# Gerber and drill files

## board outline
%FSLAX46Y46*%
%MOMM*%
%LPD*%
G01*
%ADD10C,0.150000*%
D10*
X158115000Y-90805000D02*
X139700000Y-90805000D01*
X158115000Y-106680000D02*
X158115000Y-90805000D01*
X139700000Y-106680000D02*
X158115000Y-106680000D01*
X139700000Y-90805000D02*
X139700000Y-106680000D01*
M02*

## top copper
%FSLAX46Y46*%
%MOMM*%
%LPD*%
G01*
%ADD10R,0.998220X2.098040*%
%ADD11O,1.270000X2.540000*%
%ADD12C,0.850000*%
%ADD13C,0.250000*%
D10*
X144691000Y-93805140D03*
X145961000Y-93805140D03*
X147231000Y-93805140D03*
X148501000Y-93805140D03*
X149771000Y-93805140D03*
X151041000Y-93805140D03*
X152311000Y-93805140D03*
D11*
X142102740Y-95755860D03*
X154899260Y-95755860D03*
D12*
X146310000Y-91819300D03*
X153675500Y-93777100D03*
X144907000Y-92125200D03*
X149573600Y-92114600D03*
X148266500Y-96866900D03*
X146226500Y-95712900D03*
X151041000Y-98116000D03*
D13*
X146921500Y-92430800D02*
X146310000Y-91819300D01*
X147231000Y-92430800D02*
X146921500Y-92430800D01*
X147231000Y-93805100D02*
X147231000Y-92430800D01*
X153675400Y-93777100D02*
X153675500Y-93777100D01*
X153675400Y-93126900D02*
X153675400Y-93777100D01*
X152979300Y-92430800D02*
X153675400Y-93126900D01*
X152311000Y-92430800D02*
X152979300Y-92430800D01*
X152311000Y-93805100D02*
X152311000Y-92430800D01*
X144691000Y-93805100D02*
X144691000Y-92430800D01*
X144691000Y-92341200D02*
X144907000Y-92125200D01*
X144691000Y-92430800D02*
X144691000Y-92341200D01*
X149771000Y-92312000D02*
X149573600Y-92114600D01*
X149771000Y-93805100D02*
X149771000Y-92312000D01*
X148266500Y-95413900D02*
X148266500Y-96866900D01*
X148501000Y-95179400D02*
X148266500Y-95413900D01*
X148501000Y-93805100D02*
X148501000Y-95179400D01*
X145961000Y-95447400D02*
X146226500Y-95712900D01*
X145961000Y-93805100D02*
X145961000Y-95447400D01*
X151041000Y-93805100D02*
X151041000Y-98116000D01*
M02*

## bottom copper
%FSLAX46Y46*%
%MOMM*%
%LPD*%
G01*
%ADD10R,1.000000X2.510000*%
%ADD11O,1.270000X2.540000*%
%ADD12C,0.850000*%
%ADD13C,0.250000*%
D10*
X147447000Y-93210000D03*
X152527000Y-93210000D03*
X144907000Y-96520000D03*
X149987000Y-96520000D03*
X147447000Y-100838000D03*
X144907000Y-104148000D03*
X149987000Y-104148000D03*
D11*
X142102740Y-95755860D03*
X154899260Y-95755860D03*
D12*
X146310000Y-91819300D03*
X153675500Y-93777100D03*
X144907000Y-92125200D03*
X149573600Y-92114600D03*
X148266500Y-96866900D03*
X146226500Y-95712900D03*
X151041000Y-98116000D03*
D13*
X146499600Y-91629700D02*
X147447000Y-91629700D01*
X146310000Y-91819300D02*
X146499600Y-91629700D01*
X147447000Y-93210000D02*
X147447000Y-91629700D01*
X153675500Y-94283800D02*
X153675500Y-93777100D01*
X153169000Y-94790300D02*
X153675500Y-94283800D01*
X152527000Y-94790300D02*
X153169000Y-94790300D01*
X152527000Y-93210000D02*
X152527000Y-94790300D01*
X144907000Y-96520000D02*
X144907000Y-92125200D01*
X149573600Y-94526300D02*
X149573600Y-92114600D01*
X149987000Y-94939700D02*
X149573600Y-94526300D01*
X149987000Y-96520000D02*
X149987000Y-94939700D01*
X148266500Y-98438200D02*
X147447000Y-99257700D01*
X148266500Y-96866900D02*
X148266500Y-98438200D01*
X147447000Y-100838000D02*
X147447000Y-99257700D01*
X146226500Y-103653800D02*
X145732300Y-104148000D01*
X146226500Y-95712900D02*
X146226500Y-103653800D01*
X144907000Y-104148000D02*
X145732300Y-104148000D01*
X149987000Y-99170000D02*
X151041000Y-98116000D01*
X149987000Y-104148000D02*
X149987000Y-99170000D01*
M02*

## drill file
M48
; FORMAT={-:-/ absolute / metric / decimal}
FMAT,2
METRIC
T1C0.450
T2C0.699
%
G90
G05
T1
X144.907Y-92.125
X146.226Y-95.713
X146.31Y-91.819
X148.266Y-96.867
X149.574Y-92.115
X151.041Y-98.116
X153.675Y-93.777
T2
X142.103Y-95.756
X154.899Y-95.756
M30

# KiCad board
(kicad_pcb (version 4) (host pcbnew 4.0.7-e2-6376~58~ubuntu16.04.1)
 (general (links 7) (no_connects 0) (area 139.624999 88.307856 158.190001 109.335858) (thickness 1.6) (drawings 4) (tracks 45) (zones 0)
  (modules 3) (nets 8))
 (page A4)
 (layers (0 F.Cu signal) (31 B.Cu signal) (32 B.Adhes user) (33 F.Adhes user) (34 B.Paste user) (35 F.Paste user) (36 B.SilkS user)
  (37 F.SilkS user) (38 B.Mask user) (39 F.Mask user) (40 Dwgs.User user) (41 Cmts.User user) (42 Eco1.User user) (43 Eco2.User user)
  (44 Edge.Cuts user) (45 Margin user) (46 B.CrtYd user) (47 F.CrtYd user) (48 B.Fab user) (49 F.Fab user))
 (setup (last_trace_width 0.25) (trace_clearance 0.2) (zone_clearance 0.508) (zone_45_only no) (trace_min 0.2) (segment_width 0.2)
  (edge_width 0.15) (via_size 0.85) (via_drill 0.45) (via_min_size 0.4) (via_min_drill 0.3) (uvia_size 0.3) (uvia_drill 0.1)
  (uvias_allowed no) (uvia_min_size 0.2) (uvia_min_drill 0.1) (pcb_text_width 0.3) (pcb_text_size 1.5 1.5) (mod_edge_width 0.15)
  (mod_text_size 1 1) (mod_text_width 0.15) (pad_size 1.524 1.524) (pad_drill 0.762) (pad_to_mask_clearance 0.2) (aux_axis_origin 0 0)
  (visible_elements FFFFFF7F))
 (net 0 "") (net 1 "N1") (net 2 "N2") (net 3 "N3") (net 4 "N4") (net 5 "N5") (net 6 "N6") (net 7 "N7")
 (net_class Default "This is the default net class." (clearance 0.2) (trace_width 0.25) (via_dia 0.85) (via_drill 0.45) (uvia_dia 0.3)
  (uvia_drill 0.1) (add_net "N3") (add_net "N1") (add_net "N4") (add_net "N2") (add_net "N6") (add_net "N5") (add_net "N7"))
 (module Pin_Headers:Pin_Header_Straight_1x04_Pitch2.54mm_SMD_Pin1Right (layer B.Cu) (at 148.717 94.865 270)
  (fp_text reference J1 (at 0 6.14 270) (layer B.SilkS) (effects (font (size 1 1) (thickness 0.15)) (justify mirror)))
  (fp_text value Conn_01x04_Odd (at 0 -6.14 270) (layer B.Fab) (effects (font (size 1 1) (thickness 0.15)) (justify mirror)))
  (pad 2 smd rect (at -1.655 1.27 270) (size 2.51 1) (layers B.Cu B.Paste B.Mask) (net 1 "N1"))
  (pad 4 smd rect (at -1.655 -3.81 270) (size 2.51 1) (layers B.Cu B.Paste B.Mask) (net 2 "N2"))
  (pad 1 smd rect (at 1.655 3.81 270) (size 2.51 1) (layers B.Cu B.Paste B.Mask) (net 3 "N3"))
  (pad 3 smd rect (at 1.655 -1.27 270) (size 2.51 1) (layers B.Cu B.Paste B.Mask) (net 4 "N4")))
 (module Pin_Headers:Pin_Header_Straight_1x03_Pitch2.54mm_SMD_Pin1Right (layer B.Cu) (at 147.447 102.493 270)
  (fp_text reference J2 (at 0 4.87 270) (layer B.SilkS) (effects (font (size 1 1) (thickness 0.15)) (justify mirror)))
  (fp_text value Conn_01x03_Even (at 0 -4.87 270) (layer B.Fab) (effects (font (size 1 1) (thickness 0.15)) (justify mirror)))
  (pad 2 smd rect (at -1.655 0 270) (size 2.51 1) (layers B.Cu B.Paste B.Mask) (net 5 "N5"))
  (pad 1 smd rect (at 1.655 2.54 270) (size 2.51 1) (layers B.Cu B.Paste B.Mask) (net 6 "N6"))
  (pad 3 smd rect (at 1.655 -2.54 270) (size 2.51 1) (layers B.Cu B.Paste B.Mask) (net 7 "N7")))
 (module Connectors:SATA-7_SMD (layer F.Cu) (at 148.501 105.004)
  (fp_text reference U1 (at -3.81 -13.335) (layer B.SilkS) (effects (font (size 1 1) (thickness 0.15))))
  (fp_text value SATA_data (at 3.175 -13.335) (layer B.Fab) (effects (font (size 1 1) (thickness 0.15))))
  (pad 1 smd rect (at -3.81 -11.19886) (size 0.99822 2.09804) (layers F.Cu F.Paste F.Mask) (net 3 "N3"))
  (pad 2 smd rect (at -2.54 -11.19886) (size 0.99822 2.09804) (layers F.Cu F.Paste F.Mask) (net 6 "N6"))
  (pad 3 smd rect (at -1.27 -11.19886) (size 0.99822 2.09804) (layers F.Cu F.Paste F.Mask) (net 1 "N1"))
  (pad 4 smd rect (at 0 -11.19886) (size 0.99822 2.09804) (layers F.Cu F.Paste F.Mask) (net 5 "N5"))
  (pad 5 smd rect (at 1.27 -11.19886) (size 0.99822 2.09804) (layers F.Cu F.Paste F.Mask) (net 4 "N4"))
  (pad 6 smd rect (at 2.54 -11.19886) (size 0.99822 2.09804) (layers F.Cu F.Paste F.Mask) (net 7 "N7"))
  (pad 7 smd rect (at 3.81 -11.19886) (size 0.99822 2.09804) (layers F.Cu F.Paste F.Mask) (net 2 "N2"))
  (pad M1 thru_hole oval (at -6.39826 -9.24814) (size 1.27 2.54) (drill 0.6985) (layers *.Cu F.Paste F.Mask))
  (pad M2 thru_hole oval (at 6.39826 -9.24814) (size 1.27 2.54) (drill 0.6985) (layers *.Cu F.Paste F.Mask)))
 (gr_line (start 158.115 90.805) (end 139.7 90.805) (layer Edge.Cuts) (width 0.15))
 (gr_line (start 158.115 106.68) (end 158.115 90.805) (layer Edge.Cuts) (width 0.15))
 (gr_line (start 139.7 106.68) (end 158.115 106.68) (layer Edge.Cuts) (width 0.15))
 (gr_line (start 139.7 90.805) (end 139.7 106.68) (layer Edge.Cuts) (width 0.15))
 (via (at 146.31 91.8193) (size 0.85) (layers F.Cu B.Cu) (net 1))
 (segment (start 146.4996 91.6297) (end 147.447 91.6297) (width 0.25) (layer B.Cu) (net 1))
 (segment (start 146.31 91.8193) (end 146.4996 91.6297) (width 0.25) (layer B.Cu) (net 1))
 (segment (start 146.9215 92.4308) (end 146.31 91.8193) (width 0.25) (layer F.Cu) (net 1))
 (segment (start 147.231 92.4308) (end 146.9215 92.4308) (width 0.25) (layer F.Cu) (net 1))
 (segment (start 147.447 93.21) (end 147.447 91.6297) (width 0.25) (layer B.Cu) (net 1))
 (segment (start 147.231 93.8051) (end 147.231 92.4308) (width 0.25) (layer F.Cu) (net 1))
 (via (at 153.6755 93.7771) (size 0.85) (layers F.Cu B.Cu) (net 2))
 (segment (start 153.6755 94.2838) (end 153.6755 93.7771) (width 0.25) (layer B.Cu) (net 2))
 (segment (start 153.169 94.7903) (end 153.6755 94.2838) (width 0.25) (layer B.Cu) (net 2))
 (segment (start 152.527 94.7903) (end 153.169 94.7903) (width 0.25) (layer B.Cu) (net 2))
 (segment (start 153.6754 93.7771) (end 153.6755 93.7771) (width 0.25) (layer F.Cu) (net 2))
 (segment (start 153.6754 93.1269) (end 153.6754 93.7771) (width 0.25) (layer F.Cu) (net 2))
 (segment (start 152.9793 92.4308) (end 153.6754 93.1269) (width 0.25) (layer F.Cu) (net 2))
 (segment (start 152.311 92.4308) (end 152.9793 92.4308) (width 0.25) (layer F.Cu) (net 2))
 (segment (start 152.311 93.8051) (end 152.311 92.4308) (width 0.25) (layer F.Cu) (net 2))
 (segment (start 152.527 93.21) (end 152.527 94.7903) (width 0.25) (layer B.Cu) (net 2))
 (via (at 144.907 92.1252) (size 0.85) (layers F.Cu B.Cu) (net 3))
 (segment (start 144.691 93.8051) (end 144.691 92.4308) (width 0.25) (layer F.Cu) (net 3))
 (segment (start 144.907 96.52) (end 144.907 92.1252) (width 0.25) (layer B.Cu) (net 3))
 (segment (start 144.691 92.3412) (end 144.907 92.1252) (width 0.25) (layer F.Cu) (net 3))
 (segment (start 144.691 92.4308) (end 144.691 92.3412) (width 0.25) (layer F.Cu) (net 3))
 (via (at 149.5736 92.1146) (size 0.85) (layers F.Cu B.Cu) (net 4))
 (segment (start 149.5736 94.5263) (end 149.5736 92.1146) (width 0.25) (layer B.Cu) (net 4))
 (segment (start 149.987 94.9397) (end 149.5736 94.5263) (width 0.25) (layer B.Cu) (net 4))
 (segment (start 149.771 92.312) (end 149.5736 92.1146) (width 0.25) (layer F.Cu) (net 4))
 (segment (start 149.771 93.8051) (end 149.771 92.312) (width 0.25) (layer F.Cu) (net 4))
 (segment (start 149.987 96.52) (end 149.987 94.9397) (width 0.25) (layer B.Cu) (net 4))
 (via (at 148.2665 96.8669) (size 0.85) (layers F.Cu B.Cu) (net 5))
 (segment (start 148.2665 95.4139) (end 148.2665 96.8669) (width 0.25) (layer F.Cu) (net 5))
 (segment (start 148.501 95.1794) (end 148.2665 95.4139) (width 0.25) (layer F.Cu) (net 5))
 (segment (start 148.2665 98.4382) (end 147.447 99.2577) (width 0.25) (layer B.Cu) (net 5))
 (segment (start 148.2665 96.8669) (end 148.2665 98.4382) (width 0.25) (layer B.Cu) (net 5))
 (segment (start 148.501 93.8051) (end 148.501 95.1794) (width 0.25) (layer F.Cu) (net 5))
 (segment (start 147.447 100.838) (end 147.447 99.2577) (width 0.25) (layer B.Cu) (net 5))
 (via (at 146.2265 95.7129) (size 0.85) (layers F.Cu B.Cu) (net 6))
 (segment (start 145.961 95.4474) (end 146.2265 95.7129) (width 0.25) (layer F.Cu) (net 6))
 (segment (start 145.961 93.8051) (end 145.961 95.4474) (width 0.25) (layer F.Cu) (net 6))
 (segment (start 146.2265 103.6538) (end 145.7323 104.148) (width 0.25) (layer B.Cu) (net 6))
 (segment (start 146.2265 95.7129) (end 146.2265 103.6538) (width 0.25) (layer B.Cu) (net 6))
 (segment (start 144.907 104.148) (end 145.7323 104.148) (width 0.25) (layer B.Cu) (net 6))
 (via (at 151.041 98.116) (size 0.85) (layers F.Cu B.Cu) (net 7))
 (segment (start 149.987 99.17) (end 151.041 98.116) (width 0.25) (layer B.Cu) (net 7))
 (segment (start 149.987 104.148) (end 149.987 99.17) (width 0.25) (layer B.Cu) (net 7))
 (segment (start 151.041 93.8051) (end 151.041 98.116) (width 0.25) (layer F.Cu) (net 7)))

